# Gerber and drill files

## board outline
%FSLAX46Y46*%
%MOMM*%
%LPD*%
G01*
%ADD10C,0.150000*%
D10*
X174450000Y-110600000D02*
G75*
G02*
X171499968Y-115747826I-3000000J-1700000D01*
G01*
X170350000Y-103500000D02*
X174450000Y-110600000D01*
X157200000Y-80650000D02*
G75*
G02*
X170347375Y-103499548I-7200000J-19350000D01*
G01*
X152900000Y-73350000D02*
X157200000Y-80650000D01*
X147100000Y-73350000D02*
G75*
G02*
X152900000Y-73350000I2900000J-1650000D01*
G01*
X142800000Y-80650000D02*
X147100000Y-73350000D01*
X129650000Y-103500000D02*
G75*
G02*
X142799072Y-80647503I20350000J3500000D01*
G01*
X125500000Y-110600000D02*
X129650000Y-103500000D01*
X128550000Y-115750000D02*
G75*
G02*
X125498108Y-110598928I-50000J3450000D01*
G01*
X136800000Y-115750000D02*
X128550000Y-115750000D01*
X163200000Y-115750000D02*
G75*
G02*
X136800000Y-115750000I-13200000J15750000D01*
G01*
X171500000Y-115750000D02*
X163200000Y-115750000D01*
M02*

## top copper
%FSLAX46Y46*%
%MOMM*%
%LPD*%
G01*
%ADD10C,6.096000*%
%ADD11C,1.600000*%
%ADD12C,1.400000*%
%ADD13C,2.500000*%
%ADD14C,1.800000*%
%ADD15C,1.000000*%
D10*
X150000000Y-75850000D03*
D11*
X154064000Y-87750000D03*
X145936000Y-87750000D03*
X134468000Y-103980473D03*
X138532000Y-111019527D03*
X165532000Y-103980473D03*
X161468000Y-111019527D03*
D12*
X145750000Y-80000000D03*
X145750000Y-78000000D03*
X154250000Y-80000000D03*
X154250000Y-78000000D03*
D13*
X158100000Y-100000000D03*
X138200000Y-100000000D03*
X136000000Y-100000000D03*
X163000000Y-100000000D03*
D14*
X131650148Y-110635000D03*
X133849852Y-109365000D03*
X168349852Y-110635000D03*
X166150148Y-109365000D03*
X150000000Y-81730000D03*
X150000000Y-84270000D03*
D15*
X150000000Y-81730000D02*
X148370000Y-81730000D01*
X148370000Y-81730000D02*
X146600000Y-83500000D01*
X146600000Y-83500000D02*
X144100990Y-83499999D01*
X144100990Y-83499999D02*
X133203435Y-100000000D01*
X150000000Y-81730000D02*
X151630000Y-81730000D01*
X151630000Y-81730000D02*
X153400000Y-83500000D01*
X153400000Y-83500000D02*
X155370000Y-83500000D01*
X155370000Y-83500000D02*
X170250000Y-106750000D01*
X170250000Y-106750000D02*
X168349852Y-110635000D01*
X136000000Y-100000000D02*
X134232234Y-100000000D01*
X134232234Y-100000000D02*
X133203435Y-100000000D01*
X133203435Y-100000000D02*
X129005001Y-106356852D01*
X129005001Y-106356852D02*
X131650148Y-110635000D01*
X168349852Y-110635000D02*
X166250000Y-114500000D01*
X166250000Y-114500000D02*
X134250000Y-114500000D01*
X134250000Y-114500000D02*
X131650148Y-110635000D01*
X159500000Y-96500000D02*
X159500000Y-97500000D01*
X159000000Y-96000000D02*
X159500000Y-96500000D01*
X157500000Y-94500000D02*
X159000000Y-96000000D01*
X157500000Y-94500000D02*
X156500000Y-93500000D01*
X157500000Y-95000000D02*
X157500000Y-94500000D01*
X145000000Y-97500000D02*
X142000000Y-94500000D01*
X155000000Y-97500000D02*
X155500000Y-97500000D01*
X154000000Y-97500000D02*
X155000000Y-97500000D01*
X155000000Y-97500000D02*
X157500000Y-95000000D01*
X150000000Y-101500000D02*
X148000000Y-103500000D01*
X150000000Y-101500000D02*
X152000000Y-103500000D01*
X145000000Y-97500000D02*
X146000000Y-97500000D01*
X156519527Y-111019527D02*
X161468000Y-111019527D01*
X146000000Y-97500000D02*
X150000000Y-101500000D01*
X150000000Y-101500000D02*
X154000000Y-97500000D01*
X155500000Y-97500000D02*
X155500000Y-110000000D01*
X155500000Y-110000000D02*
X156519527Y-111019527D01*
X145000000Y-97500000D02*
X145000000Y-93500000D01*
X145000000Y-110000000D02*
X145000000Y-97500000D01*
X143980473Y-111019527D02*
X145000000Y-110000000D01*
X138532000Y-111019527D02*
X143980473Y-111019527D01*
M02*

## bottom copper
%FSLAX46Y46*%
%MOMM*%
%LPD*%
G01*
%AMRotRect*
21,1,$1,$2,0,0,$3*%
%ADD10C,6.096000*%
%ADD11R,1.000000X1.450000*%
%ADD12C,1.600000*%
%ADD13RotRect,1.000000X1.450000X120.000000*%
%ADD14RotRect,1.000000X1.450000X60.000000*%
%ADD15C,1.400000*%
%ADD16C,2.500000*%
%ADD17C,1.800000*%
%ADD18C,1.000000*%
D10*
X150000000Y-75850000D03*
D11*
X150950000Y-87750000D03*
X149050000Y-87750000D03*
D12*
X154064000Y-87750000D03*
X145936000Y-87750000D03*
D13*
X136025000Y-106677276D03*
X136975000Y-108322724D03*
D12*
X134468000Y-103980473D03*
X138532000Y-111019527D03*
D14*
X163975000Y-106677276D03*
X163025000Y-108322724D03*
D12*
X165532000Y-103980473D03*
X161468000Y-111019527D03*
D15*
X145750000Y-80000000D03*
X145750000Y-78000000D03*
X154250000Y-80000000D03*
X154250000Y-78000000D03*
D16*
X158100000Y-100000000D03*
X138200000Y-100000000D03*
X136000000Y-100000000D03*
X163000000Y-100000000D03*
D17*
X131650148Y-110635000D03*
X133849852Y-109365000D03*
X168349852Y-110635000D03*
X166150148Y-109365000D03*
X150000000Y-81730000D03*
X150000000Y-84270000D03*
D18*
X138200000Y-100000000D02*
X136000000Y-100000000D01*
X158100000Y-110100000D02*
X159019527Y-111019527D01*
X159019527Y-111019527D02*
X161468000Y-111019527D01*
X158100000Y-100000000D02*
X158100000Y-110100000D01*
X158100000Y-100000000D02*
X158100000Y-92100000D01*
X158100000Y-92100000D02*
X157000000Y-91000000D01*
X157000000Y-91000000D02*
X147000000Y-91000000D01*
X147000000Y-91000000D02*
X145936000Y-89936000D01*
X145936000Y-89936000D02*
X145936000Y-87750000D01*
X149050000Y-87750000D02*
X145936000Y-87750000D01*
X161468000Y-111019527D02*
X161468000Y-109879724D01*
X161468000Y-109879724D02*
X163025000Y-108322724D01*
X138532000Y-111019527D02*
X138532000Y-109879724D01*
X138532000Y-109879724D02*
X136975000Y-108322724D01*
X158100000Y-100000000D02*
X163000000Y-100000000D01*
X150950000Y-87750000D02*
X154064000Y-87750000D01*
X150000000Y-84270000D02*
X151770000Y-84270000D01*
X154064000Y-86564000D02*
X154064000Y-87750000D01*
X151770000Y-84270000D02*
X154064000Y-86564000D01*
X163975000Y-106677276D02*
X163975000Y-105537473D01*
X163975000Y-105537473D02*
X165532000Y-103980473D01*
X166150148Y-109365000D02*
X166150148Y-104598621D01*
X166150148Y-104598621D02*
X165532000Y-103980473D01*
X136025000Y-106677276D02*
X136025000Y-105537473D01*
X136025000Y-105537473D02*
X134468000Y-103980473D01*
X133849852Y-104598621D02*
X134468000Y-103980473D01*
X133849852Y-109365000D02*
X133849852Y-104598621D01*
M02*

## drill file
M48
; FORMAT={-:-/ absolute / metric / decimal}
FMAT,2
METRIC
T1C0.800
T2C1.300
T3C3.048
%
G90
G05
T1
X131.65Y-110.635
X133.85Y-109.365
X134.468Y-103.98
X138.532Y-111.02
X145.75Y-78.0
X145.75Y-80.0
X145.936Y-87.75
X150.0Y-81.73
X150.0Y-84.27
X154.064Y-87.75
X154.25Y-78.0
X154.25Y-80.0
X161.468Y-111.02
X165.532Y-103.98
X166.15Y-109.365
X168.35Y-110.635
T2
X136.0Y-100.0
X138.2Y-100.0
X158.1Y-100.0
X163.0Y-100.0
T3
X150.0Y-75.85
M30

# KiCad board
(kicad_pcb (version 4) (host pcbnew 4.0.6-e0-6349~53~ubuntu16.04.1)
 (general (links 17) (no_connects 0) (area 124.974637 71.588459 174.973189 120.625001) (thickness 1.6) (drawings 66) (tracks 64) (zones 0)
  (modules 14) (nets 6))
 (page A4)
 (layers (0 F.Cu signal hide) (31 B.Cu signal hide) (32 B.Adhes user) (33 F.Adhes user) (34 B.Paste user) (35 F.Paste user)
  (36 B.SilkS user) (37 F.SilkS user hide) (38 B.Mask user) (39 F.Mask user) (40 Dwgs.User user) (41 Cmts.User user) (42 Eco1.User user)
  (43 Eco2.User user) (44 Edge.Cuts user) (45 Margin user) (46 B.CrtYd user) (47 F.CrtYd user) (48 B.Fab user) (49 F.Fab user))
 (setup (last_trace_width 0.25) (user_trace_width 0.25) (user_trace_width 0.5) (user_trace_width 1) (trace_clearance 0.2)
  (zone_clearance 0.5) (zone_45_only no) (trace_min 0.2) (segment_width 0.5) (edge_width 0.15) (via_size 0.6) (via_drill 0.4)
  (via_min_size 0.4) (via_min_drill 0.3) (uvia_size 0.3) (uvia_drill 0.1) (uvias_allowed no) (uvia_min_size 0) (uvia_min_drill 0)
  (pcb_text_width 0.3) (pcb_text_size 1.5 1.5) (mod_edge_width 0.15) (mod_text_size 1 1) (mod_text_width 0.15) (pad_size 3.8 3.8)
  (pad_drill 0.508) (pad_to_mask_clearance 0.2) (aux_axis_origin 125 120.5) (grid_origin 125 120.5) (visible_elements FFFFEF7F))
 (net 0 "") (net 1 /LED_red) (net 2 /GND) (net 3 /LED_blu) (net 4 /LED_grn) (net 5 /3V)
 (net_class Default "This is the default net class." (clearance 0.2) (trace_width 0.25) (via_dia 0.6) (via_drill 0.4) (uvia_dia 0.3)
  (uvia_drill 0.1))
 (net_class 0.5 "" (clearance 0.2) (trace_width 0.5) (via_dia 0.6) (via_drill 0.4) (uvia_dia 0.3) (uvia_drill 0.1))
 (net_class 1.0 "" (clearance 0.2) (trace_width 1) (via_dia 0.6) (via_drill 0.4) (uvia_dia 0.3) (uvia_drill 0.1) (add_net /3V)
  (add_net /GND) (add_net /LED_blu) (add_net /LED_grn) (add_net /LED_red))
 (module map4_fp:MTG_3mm (layer F.Cu) (at 150 75.85)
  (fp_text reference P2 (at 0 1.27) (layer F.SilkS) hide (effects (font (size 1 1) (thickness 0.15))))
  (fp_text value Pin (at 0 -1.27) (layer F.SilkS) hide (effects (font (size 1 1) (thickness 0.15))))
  (pad 1 thru_hole circle (at 0 0) (size 6.096 6.096) (drill 3.048) (layers *.Cu *.Mask F.SilkS)))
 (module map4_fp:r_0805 (layer B.Cu) (at 150 87.75)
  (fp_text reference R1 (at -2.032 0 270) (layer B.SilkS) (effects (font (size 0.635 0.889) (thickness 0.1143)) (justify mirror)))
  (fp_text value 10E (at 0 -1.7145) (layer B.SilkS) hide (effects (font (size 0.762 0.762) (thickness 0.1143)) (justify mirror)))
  (pad 2 smd rect (at 0.95 0) (size 1 1.45) (layers B.Cu B.Paste B.Mask) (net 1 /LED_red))
  (pad 1 smd rect (at -0.95 0) (size 1 1.45) (layers B.Cu B.Paste B.Mask) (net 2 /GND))
  (pad 2 thru_hole circle (at 4.064 0) (size 1.6 1.6) (drill 0.8) (layers *.Cu *.Mask B.SilkS) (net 1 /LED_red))
  (pad 1 thru_hole circle (at -4.064 0) (size 1.6 1.6) (drill 0.8) (layers *.Cu *.Mask B.SilkS) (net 2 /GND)))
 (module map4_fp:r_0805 (layer B.Cu) (at 136.5 107.5 120)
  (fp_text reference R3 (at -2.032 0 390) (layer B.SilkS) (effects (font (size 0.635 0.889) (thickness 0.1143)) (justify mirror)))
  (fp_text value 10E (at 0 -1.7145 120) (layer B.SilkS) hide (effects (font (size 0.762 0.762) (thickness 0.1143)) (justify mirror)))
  (pad 2 smd rect (at 0.95 0 120) (size 1 1.45) (layers B.Cu B.Paste B.Mask) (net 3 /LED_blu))
  (pad 1 smd rect (at -0.95 0 120) (size 1 1.45) (layers B.Cu B.Paste B.Mask) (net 2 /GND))
  (pad 2 thru_hole circle (at 4.064 0 120) (size 1.6 1.6) (drill 0.8) (layers *.Cu *.Mask B.SilkS) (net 3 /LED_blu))
  (pad 1 thru_hole circle (at -4.064 0 120) (size 1.6 1.6) (drill 0.8) (layers *.Cu *.Mask B.SilkS) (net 2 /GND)))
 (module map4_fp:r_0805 (layer B.Cu) (at 163.5 107.5 60)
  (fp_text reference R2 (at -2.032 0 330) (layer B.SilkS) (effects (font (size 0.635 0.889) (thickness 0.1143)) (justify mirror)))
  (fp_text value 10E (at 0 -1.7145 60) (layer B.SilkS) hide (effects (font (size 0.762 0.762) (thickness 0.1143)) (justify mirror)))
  (pad 2 smd rect (at 0.95 0 60) (size 1 1.45) (layers B.Cu B.Paste B.Mask) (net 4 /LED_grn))
  (pad 1 smd rect (at -0.95 0 60) (size 1 1.45) (layers B.Cu B.Paste B.Mask) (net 2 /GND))
  (pad 2 thru_hole circle (at 4.064 0 60) (size 1.6 1.6) (drill 0.8) (layers *.Cu *.Mask B.SilkS) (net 4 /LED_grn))
  (pad 1 thru_hole circle (at -4.064 0 60) (size 1.6 1.6) (drill 0.8) (layers *.Cu *.Mask B.SilkS) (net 2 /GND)))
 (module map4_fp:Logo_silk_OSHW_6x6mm (layer B.Cu) (at 150 107.5 180)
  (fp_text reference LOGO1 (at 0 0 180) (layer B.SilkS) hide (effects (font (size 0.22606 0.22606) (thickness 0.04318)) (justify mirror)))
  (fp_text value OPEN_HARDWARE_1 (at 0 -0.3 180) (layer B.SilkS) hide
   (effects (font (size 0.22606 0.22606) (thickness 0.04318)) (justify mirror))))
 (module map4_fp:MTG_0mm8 (layer F.Cu) (at 145.75 80)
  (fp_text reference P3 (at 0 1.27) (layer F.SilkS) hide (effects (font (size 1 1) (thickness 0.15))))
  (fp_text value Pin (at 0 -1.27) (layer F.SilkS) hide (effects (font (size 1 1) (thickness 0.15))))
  (pad 1 thru_hole circle (at 0 0) (size 1.4 1.4) (drill 0.8) (layers *.Cu *.Mask F.SilkS)))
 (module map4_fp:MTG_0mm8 (layer F.Cu) (at 145.75 78)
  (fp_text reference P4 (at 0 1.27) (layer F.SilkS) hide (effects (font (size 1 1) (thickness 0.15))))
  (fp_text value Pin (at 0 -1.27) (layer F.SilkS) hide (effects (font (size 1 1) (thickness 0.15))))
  (pad 1 thru_hole circle (at 0 0) (size 1.4 1.4) (drill 0.8) (layers *.Cu *.Mask F.SilkS)))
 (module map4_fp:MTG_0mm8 (layer F.Cu) (at 154.25 80)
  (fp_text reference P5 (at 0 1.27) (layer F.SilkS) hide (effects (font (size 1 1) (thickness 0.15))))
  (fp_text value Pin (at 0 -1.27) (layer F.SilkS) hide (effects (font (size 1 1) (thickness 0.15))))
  (pad 1 thru_hole circle (at 0 0) (size 1.4 1.4) (drill 0.8) (layers *.Cu *.Mask F.SilkS)))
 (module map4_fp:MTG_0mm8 (layer F.Cu) (at 154.25 78)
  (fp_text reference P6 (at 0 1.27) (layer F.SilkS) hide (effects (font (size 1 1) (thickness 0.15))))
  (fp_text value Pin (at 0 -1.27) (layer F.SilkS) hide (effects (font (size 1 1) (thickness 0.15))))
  (pad 1 thru_hole circle (at 0 0) (size 1.4 1.4) (drill 0.8) (layers *.Cu *.Mask F.SilkS)))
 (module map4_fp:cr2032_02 (layer B.Cu) (at 150 100 90)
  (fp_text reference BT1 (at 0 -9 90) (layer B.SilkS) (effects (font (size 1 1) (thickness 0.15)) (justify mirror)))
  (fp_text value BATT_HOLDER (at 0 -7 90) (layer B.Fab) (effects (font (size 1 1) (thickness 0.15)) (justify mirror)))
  (pad 2 thru_hole circle (at 0 8.1 90) (size 2.5 2.5) (drill 1.3) (layers *.Cu *.Mask B.SilkS) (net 2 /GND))
  (pad 1 thru_hole circle (at 0 -11.8 90) (size 2.5 2.5) (drill 1.3) (layers *.Cu *.Mask B.SilkS) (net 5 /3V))
  (pad 1 thru_hole circle (at 0 -14 90) (size 2.5 2.5) (drill 1.3) (layers *.Cu *.Mask B.SilkS) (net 5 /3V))
  (pad 2 thru_hole circle (at 0 13 90) (size 2.5 2.5) (drill 1.3) (layers *.Cu *.Mask B.SilkS) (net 2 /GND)))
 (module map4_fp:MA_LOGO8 (layer F.Cu) (at 150 96)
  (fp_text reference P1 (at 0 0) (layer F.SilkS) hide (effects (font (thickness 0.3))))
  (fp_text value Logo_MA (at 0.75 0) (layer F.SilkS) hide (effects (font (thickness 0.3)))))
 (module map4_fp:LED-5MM (layer F.Cu) (at 132.75 110 30)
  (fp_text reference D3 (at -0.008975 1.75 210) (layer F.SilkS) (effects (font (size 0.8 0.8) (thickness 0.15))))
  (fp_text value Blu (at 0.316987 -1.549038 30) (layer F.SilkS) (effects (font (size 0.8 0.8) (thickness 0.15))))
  (pad 1 thru_hole circle (at -1.27 0 30) (size 1.8 1.8) (drill 0.8) (layers *.Cu *.Mask F.SilkS) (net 5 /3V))
  (pad 2 thru_hole circle (at 1.27 0 30) (size 1.8 1.8) (drill 0.8) (layers *.Cu *.Mask F.SilkS) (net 3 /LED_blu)))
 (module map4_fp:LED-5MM (layer F.Cu) (at 167.25 110 150)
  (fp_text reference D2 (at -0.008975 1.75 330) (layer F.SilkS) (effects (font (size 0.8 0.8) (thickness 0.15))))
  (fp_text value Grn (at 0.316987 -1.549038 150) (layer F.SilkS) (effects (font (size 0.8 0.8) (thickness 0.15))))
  (pad 1 thru_hole circle (at -1.27 0 150) (size 1.8 1.8) (drill 0.8) (layers *.Cu *.Mask F.SilkS) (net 5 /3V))
  (pad 2 thru_hole circle (at 1.27 0 150) (size 1.8 1.8) (drill 0.8) (layers *.Cu *.Mask F.SilkS) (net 4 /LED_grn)))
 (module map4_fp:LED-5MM (layer F.Cu) (at 150 83 270)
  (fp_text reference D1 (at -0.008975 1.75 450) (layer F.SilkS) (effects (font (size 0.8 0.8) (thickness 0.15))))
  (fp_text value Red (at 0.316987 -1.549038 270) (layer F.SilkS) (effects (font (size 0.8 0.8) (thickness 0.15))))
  (pad 1 thru_hole circle (at -1.27 0 270) (size 1.8 1.8) (drill 0.8) (layers *.Cu *.Mask F.SilkS) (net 5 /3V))
  (pad 2 thru_hole circle (at 1.27 0 270) (size 1.8 1.8) (drill 0.8) (layers *.Cu *.Mask F.SilkS) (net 1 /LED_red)))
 (gr_arc (start 171.45 112.3) (end 174.45 110.6) (angle 118.7084745) (layer Edge.Cuts) (width 0.15))
 (gr_line (start 170.35 103.5) (end 174.45 110.6) (layer Edge.Cuts) (width 0.15))
 (gr_arc (start 150 100) (end 157.2 80.65) (angle 79.34895054) (layer Edge.Cuts) (width 0.15))
 (gr_line (start 152.9 73.35) (end 157.2 80.65) (layer Edge.Cuts) (width 0.15))
 (gr_arc (start 150 75) (end 147.1 73.35) (angle 120.7232391) (layer Edge.Cuts) (width 0.15))
 (gr_line (start 142.8 80.65) (end 147.1 73.35) (layer Edge.Cuts) (width 0.15))
 (gr_arc (start 150 100) (end 129.65 103.5) (angle 79.34895344) (layer Edge.Cuts) (width 0.15))
 (gr_line (start 125.5 110.6) (end 129.65 103.5) (layer Edge.Cuts) (width 0.15))
 (gr_arc (start 128.5 112.3) (end 128.55 115.75) (angle 120.3690896) (layer Edge.Cuts) (width 0.15))
 (gr_line (start 136.8 115.75) (end 128.55 115.75) (layer Edge.Cuts) (width 0.15))
 (gr_arc (start 150 100) (end 163.2 115.75) (angle 79.93242788) (layer Edge.Cuts) (width 0.15))
 (gr_line (start 171.5 115.75) (end 163.2 115.75) (layer Edge.Cuts) (width 0.15))
 (segment (start 150 81.73) (end 148.37 81.73) (width 1) (layer F.Cu) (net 5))
 (segment (start 148.37 81.73) (end 146.6 83.5) (width 1) (layer F.Cu) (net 5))
 (segment (start 146.6 83.5) (end 144.10099 83.499999) (width 1) (layer F.Cu) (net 5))
 (segment (start 144.10099 83.499999) (end 133.203435 100) (width 1) (layer F.Cu) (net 5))
 (segment (start 150 81.73) (end 151.63 81.73) (width 1) (layer F.Cu) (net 5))
 (segment (start 151.63 81.73) (end 153.4 83.5) (width 1) (layer F.Cu) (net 5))
 (segment (start 153.4 83.5) (end 155.37 83.5) (width 1) (layer F.Cu) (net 5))
 (segment (start 155.37 83.5) (end 170.25 106.75) (width 1) (layer F.Cu) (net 5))
 (segment (start 170.25 106.75) (end 168.349852 110.635) (width 1) (layer F.Cu) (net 5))
 (segment (start 136 100) (end 134.232234 100) (width 1) (layer F.Cu) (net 5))
 (segment (start 134.232234 100) (end 133.203435 100) (width 1) (layer F.Cu) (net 5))
 (segment (start 133.203435 100) (end 129.005001 106.356852) (width 1) (layer F.Cu) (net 5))
 (segment (start 138.2 100) (end 136 100) (width 1) (layer B.Cu) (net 5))
 (segment (start 129.005001 106.356852) (end 131.650148 110.635) (width 1) (layer F.Cu) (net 5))
 (segment (start 168.349852 110.635) (end 166.25 114.5) (width 1) (layer F.Cu) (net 5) (status 10))
 (segment (start 166.25 114.5) (end 134.25 114.5) (width 1) (layer F.Cu) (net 5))
 (segment (start 134.25 114.5) (end 131.650148 110.635) (width 1) (layer F.Cu) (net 5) (status 20))
 (segment (start 159.5 96.5) (end 159.5 97.5) (width 1) (layer F.Cu) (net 2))
 (segment (start 159 96) (end 159.5 96.5) (width 1) (layer F.Cu) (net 2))
 (segment (start 157.5 94.5) (end 159 96) (width 1) (layer F.Cu) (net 2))
 (segment (start 157.5 94.5) (end 156.5 93.5) (width 1) (layer F.Cu) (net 2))
 (segment (start 157.5 95) (end 157.5 94.5) (width 1) (layer F.Cu) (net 2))
 (segment (start 145 97.5) (end 142 94.5) (width 1) (layer F.Cu) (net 2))
 (segment (start 155 97.5) (end 155.5 97.5) (width 1) (layer F.Cu) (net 2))
 (segment (start 154 97.5) (end 155 97.5) (width 1) (layer F.Cu) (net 2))
 (segment (start 155 97.5) (end 157.5 95) (width 1) (layer F.Cu) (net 2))
 (segment (start 150 101.5) (end 148 103.5) (width 1) (layer F.Cu) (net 2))
 (segment (start 150 101.5) (end 152 103.5) (width 1) (layer F.Cu) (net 2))
 (segment (start 145 97.5) (end 146 97.5) (width 1) (layer F.Cu) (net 2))
 (segment (start 156.519527 111.019527) (end 161.468 111.019527) (width 1) (layer F.Cu) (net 2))
 (segment (start 146 97.5) (end 150 101.5) (width 1) (layer F.Cu) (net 2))
 (segment (start 150 101.5) (end 154 97.5) (width 1) (layer F.Cu) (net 2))
 (segment (start 155.5 97.5) (end 155.5 110) (width 1) (layer F.Cu) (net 2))
 (segment (start 155.5 110) (end 156.519527 111.019527) (width 1) (layer F.Cu) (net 2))
 (segment (start 145 97.5) (end 145 93.5) (width 1) (layer F.Cu) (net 2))
 (segment (start 145 110) (end 145 97.5) (width 1) (layer F.Cu) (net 2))
 (segment (start 143.980473 111.019527) (end 145 110) (width 1) (layer F.Cu) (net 2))
 (segment (start 138.532 111.019527) (end 143.980473 111.019527) (width 1) (layer F.Cu) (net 2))
 (segment (start 158.1 110.1) (end 159.019527 111.019527) (width 1) (layer B.Cu) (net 2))
 (segment (start 159.019527 111.019527) (end 161.468 111.019527) (width 1) (layer B.Cu) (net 2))
 (segment (start 158.1 100) (end 158.1 110.1) (width 1) (layer B.Cu) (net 2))
 (segment (start 158.1 100) (end 158.1 92.1) (width 1) (layer B.Cu) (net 2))
 (segment (start 158.1 92.1) (end 157 91) (width 1) (layer B.Cu) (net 2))
 (segment (start 157 91) (end 147 91) (width 1) (layer B.Cu) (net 2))
 (segment (start 147 91) (end 145.936 89.936) (width 1) (layer B.Cu) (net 2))
 (segment (start 145.936 89.936) (end 145.936 87.75) (width 1) (layer B.Cu) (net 2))
 (segment (start 149.05 87.75) (end 145.936 87.75) (width 1) (layer B.Cu) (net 2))
 (segment (start 161.468 111.019527) (end 161.468 109.879724) (width 1) (layer B.Cu) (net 2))
 (segment (start 161.468 109.879724) (end 163.025 108.322724) (width 1) (layer B.Cu) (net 2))
 (segment (start 138.532 111.019527) (end 138.532 109.879724) (width 1) (layer B.Cu) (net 2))
 (segment (start 138.532 109.879724) (end 136.975 108.322724) (width 1) (layer B.Cu) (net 2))
 (segment (start 158.1 100) (end 163 100) (width 1) (layer B.Cu) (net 2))
 (segment (start 150.95 87.75) (end 154.064 87.75) (width 1) (layer B.Cu) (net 1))
 (segment (start 150 84.27) (end 151.77 84.27) (width 1) (layer B.Cu) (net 1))
 (segment (start 154.064 86.564) (end 154.064 87.75) (width 1) (layer B.Cu) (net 1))
 (segment (start 151.77 84.27) (end 154.064 86.564) (width 1) (layer B.Cu) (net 1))
 (segment (start 163.975 106.677276) (end 163.975 105.537473) (width 1) (layer B.Cu) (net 4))
 (segment (start 163.975 105.537473) (end 165.532 103.980473) (width 1) (layer B.Cu) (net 4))
 (segment (start 166.150148 109.365) (end 166.150148 104.598621) (width 1) (layer B.Cu) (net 4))
 (segment (start 166.150148 104.598621) (end 165.532 103.980473) (width 1) (layer B.Cu) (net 4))
 (segment (start 136.025 106.677276) (end 136.025 105.537473) (width 1) (layer B.Cu) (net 3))
 (segment (start 136.025 105.537473) (end 134.468 103.980473) (width 1) (layer B.Cu) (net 3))
 (segment (start 133.849852 104.598621) (end 134.468 103.980473) (width 1) (layer B.Cu) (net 3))
 (segment (start 133.849852 109.365) (end 133.849852 104.598621) (width 1) (layer B.Cu) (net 3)))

